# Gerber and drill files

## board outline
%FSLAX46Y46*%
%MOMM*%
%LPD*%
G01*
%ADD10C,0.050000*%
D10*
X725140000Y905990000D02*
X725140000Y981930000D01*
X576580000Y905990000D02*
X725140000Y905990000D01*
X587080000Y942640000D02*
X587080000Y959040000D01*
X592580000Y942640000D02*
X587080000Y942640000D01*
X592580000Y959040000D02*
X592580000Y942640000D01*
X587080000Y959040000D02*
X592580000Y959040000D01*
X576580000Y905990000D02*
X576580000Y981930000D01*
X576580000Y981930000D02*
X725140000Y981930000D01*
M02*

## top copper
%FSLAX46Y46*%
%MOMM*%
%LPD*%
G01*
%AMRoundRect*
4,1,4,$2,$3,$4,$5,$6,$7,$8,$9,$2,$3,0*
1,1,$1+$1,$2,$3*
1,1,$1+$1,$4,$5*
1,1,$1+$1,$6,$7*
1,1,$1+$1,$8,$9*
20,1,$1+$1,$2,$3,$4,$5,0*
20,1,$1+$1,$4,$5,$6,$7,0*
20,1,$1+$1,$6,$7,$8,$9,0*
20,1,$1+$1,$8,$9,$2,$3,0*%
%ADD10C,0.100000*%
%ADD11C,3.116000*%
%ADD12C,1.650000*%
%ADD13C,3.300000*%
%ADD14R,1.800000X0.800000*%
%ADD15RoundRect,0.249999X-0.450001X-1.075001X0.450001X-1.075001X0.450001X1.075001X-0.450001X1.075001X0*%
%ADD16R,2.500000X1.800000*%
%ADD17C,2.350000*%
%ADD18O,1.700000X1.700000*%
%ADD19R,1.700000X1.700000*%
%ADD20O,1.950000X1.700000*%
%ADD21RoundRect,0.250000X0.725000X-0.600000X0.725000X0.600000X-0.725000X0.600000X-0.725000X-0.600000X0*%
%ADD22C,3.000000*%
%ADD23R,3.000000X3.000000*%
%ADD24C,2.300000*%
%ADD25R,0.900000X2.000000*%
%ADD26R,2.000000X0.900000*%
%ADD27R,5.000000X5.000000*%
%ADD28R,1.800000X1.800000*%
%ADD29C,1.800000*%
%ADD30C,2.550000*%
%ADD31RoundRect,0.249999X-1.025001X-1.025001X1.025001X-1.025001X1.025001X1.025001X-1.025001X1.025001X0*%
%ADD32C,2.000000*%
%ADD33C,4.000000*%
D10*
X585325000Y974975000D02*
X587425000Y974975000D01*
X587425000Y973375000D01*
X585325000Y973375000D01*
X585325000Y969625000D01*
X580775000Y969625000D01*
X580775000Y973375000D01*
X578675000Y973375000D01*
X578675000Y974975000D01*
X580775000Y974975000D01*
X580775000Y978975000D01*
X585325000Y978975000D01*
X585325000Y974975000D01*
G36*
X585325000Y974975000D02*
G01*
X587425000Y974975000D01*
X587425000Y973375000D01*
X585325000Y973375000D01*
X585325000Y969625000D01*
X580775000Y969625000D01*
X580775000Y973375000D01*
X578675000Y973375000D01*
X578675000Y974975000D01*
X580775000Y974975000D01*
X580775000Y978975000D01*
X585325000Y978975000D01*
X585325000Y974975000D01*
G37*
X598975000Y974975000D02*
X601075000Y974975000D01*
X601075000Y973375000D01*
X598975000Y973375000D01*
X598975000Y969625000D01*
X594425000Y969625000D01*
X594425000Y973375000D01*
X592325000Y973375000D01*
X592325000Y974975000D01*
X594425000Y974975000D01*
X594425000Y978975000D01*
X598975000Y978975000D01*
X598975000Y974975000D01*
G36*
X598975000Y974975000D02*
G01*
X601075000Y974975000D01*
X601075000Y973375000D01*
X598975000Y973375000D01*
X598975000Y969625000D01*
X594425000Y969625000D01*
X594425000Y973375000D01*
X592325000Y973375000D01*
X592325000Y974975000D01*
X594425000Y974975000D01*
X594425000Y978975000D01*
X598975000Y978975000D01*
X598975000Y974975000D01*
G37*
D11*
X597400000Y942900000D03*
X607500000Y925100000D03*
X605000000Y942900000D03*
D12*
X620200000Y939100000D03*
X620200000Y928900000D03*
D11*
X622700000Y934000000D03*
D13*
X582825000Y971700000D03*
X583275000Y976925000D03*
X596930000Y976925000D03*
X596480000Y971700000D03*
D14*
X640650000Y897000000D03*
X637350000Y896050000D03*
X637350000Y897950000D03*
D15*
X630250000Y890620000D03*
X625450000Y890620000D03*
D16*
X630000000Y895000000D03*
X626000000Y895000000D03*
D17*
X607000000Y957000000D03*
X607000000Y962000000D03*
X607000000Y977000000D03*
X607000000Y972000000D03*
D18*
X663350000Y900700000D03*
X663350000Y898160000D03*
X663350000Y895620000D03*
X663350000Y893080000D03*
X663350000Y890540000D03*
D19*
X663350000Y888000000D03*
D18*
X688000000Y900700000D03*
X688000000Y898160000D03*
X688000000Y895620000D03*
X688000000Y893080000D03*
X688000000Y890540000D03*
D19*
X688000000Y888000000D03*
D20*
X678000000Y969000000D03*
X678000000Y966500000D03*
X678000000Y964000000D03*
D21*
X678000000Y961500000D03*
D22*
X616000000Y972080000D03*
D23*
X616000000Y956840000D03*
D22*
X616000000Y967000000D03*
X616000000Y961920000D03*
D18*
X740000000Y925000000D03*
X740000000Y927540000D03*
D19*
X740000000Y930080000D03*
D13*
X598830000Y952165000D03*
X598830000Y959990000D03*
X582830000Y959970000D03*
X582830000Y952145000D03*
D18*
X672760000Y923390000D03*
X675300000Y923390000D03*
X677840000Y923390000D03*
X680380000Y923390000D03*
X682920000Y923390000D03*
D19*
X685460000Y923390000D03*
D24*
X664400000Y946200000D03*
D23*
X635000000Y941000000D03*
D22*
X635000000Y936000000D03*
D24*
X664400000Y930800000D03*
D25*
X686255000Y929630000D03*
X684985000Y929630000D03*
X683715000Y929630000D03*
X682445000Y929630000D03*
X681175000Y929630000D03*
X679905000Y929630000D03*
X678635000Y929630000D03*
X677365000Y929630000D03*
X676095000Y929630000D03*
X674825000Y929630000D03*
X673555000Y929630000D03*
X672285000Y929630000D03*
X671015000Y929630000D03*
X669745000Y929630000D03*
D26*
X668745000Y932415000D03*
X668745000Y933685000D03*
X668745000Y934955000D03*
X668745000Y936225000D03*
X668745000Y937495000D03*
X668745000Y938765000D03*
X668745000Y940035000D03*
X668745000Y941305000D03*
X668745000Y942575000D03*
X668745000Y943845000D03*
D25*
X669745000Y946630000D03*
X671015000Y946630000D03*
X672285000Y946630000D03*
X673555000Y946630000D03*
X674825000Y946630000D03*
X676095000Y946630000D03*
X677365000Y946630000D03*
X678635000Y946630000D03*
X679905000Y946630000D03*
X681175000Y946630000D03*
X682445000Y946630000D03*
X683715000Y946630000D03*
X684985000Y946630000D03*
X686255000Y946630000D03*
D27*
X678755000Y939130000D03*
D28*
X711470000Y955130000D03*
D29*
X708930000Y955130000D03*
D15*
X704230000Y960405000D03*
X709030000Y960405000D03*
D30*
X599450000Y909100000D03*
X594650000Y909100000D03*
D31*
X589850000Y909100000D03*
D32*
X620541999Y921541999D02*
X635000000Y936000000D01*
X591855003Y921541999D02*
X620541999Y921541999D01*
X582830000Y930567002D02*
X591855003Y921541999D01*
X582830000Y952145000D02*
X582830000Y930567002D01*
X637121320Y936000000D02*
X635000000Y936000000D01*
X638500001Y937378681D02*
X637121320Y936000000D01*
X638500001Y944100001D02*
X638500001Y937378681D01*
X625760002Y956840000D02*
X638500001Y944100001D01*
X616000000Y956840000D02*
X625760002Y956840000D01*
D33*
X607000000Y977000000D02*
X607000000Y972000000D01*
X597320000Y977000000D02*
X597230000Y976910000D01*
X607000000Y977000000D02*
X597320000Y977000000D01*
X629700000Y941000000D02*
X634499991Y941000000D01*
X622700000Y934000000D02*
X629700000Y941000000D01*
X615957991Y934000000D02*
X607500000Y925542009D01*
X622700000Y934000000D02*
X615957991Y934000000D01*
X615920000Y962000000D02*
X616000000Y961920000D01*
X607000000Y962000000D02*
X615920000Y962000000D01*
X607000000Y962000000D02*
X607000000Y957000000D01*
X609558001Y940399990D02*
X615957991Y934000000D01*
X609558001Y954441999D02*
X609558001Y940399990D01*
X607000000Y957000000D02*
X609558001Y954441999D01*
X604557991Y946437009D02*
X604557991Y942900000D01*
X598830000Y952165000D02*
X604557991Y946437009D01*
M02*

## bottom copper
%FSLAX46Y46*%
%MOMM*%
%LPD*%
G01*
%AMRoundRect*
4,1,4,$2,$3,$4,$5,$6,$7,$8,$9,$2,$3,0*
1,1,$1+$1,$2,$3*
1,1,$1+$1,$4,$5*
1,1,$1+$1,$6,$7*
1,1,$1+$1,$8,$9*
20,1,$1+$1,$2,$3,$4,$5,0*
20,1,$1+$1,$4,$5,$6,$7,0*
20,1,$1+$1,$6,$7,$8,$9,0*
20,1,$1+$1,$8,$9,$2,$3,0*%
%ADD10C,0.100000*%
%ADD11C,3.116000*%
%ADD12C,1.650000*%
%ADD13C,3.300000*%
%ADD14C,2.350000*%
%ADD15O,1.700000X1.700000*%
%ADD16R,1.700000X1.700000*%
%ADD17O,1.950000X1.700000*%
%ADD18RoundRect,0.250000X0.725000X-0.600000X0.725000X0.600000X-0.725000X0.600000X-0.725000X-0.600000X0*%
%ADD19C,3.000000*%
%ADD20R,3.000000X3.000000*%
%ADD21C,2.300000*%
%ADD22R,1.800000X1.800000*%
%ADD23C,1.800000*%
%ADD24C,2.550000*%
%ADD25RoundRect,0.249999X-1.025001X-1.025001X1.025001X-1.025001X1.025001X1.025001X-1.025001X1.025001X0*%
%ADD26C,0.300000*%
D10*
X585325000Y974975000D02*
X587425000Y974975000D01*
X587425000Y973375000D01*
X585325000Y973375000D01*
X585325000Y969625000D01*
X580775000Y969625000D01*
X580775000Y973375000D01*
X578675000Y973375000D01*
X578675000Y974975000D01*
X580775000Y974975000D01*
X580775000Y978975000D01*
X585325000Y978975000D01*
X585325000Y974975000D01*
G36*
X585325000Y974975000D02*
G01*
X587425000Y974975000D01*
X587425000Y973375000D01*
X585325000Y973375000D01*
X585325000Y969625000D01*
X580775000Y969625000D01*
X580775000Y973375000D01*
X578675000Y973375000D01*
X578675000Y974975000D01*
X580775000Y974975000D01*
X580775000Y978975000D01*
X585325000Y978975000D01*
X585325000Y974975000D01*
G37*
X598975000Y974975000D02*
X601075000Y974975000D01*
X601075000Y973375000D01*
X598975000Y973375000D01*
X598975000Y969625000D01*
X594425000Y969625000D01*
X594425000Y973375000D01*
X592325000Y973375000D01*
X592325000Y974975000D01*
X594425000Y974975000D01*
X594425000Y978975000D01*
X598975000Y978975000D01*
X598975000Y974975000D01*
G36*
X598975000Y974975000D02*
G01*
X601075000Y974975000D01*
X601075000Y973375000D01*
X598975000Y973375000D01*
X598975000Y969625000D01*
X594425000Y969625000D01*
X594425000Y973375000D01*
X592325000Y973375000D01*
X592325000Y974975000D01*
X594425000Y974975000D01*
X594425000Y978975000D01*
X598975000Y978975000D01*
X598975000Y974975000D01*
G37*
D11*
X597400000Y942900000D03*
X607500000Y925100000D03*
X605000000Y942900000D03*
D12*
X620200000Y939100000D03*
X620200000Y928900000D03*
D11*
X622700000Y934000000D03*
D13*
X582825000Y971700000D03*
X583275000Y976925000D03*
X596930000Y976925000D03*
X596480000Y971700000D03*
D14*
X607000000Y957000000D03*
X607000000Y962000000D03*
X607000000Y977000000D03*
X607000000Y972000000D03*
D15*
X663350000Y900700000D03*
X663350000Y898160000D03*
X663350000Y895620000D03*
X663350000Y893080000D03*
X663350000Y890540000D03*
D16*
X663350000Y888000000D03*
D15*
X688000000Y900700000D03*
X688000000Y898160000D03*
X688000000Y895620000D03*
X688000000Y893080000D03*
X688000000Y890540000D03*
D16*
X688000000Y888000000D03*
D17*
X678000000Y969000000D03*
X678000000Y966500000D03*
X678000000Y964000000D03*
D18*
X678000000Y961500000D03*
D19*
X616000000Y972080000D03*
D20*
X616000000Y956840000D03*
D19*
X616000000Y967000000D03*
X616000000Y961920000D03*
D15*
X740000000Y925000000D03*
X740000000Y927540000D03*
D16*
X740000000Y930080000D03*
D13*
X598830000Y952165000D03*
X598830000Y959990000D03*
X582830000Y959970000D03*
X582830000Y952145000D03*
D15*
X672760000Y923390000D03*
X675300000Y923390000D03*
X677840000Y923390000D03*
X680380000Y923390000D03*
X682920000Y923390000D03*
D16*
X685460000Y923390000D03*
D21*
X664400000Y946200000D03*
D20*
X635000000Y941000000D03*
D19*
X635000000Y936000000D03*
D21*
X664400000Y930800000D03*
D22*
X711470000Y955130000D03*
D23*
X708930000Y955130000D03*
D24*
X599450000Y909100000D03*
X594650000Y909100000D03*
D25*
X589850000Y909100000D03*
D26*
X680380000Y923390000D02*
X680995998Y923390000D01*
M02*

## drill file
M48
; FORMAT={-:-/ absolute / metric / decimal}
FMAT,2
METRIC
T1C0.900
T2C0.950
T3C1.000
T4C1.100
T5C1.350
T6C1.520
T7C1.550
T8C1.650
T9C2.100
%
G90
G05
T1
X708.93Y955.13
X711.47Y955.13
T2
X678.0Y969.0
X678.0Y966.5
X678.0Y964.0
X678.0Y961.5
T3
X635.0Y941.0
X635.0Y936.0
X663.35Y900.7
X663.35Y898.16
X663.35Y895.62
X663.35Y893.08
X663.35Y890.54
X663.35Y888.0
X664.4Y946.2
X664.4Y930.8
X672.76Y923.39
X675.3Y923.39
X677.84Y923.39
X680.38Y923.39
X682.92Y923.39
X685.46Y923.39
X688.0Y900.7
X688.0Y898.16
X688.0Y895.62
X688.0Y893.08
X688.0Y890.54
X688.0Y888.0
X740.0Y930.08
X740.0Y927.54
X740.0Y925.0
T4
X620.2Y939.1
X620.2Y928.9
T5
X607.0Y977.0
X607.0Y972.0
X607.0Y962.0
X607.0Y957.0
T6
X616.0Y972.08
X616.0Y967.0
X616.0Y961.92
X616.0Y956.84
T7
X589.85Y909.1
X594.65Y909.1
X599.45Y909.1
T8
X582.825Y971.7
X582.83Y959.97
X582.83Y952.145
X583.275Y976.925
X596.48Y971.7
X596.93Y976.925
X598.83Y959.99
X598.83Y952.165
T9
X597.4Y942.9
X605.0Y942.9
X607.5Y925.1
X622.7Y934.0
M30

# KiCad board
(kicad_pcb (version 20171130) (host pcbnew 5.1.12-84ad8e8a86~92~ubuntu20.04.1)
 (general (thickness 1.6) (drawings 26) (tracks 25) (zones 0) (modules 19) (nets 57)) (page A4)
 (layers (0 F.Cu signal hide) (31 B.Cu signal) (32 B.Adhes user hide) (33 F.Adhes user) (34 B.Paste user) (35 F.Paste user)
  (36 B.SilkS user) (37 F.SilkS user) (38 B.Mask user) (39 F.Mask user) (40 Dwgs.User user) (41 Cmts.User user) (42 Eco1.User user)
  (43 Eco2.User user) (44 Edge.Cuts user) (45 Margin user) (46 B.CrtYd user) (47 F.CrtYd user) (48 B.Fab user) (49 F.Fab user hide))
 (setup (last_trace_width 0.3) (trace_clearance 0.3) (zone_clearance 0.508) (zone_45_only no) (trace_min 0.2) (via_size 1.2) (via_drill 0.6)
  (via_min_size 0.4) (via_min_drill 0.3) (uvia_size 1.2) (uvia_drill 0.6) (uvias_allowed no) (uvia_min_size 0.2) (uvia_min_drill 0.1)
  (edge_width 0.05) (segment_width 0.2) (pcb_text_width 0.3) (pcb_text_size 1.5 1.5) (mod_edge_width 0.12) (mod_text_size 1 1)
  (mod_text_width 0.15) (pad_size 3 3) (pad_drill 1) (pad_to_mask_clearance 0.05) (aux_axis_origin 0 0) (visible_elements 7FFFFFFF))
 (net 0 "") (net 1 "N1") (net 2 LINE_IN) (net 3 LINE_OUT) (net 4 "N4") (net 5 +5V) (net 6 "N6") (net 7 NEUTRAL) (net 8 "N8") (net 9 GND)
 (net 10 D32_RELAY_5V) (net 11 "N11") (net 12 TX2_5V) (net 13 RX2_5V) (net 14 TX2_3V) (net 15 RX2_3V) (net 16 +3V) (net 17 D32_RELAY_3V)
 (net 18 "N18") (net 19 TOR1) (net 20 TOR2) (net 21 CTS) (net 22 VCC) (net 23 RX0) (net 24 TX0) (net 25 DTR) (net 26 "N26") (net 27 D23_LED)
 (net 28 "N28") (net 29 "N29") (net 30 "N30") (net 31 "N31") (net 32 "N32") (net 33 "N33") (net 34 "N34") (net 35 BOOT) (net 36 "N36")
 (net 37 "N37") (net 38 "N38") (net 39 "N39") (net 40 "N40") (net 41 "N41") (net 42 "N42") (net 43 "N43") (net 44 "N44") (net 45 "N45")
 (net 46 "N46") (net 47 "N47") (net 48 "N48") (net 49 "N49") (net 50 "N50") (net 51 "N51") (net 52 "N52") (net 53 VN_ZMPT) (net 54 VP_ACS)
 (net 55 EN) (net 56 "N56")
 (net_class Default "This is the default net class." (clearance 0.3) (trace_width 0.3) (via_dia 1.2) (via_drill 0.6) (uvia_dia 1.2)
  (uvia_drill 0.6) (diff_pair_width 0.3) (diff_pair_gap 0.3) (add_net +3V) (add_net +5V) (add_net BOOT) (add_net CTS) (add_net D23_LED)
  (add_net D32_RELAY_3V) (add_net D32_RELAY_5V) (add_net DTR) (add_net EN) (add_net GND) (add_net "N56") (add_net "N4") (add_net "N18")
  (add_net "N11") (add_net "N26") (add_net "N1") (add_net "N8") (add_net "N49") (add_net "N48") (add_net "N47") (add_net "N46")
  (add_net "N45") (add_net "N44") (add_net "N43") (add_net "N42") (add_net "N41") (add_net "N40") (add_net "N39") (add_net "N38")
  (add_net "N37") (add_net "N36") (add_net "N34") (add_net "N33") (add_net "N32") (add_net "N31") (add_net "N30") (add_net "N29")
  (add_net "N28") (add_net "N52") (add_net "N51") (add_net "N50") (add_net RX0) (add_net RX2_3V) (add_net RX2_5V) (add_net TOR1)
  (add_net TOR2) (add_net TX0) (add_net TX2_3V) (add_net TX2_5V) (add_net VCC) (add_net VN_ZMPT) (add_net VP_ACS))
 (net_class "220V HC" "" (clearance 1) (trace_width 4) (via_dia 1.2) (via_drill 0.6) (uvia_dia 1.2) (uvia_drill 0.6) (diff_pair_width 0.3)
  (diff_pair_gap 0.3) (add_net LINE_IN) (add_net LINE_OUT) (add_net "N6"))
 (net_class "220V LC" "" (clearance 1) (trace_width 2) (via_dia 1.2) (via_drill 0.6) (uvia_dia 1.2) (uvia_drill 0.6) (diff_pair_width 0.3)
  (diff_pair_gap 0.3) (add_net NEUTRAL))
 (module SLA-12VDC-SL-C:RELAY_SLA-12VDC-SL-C (layer F.Cu) (at 605 -934 90)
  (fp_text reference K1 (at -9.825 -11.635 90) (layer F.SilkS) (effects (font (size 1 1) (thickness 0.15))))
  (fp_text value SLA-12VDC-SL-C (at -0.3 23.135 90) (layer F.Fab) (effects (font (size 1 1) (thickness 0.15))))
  (pad NC thru_hole circle (at 8.9 -7.6 90) (size 3.116 3.116) (drill 2.1) (layers *.Cu *.Mask) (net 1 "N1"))
  (pad COM2 thru_hole circle (at -8.9 2.5 90) (size 3.116 3.116) (drill 2.1) (layers *.Cu *.Mask) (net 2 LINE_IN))
  (pad NO thru_hole circle (at 8.9 0 90) (size 3.116 3.116) (drill 2.1) (layers *.Cu *.Mask) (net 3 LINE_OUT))
  (pad C2 thru_hole circle (at 5.1 15.2 90) (size 1.65 1.65) (drill 1.1) (layers *.Cu *.Mask) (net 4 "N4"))
  (pad C1 thru_hole circle (at -5.1 15.2 90) (size 1.65 1.65) (drill 1.1) (layers *.Cu *.Mask) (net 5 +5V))
  (pad COM1 thru_hole circle (at 0 17.7 90) (size 3.116 3.116) (drill 2.1) (layers *.Cu *.Mask) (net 2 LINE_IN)))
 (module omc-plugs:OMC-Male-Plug (layer F.Cu) (at 583 -974)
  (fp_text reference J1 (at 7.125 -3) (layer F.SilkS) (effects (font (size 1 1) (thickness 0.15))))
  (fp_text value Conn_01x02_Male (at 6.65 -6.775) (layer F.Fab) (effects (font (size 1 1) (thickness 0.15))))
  (fp_poly
   (pts (xy 2.325 -0.975) (xy 4.425 -0.975) (xy 4.425 0.625) (xy 2.325 0.625) (xy 2.325 4.375) (xy -2.225 4.375) (xy -2.225 0.625)
    (xy -4.325 0.625) (xy -4.325 -0.975) (xy -2.225 -0.975) (xy -2.225 -4.975) (xy 2.325 -4.975))
   (layer F.Cu) (width 0.1))
  (fp_poly
   (pts (xy 2.325 -0.975) (xy 4.425 -0.975) (xy 4.425 0.625) (xy 2.325 0.625) (xy 2.325 4.375) (xy -2.225 4.375) (xy -2.225 0.625)
    (xy -4.325 0.625) (xy -4.325 -0.975) (xy -2.225 -0.975) (xy -2.225 -4.975) (xy 2.325 -4.975))
   (layer B.Cu) (width 0.1))
  (fp_poly
   (pts (xy 15.975 -0.975) (xy 18.075 -0.975) (xy 18.075 0.625) (xy 15.975 0.625) (xy 15.975 4.375) (xy 11.425 4.375) (xy 11.425 0.625)
    (xy 9.325 0.625) (xy 9.325 -0.975) (xy 11.425 -0.975) (xy 11.425 -4.975) (xy 15.975 -4.975))
   (layer B.Cu) (width 0.1))
  (fp_poly
   (pts (xy 15.975 -0.975) (xy 18.075 -0.975) (xy 18.075 0.625) (xy 15.975 0.625) (xy 15.975 4.375) (xy 11.425 4.375) (xy 11.425 0.625)
    (xy 9.325 0.625) (xy 9.325 -0.975) (xy 11.425 -0.975) (xy 11.425 -4.975) (xy 15.975 -4.975))
   (layer F.Cu) (width 0.1))
  (pad 1 thru_hole circle (at -0.175 2.3) (size 3.3 3.3) (drill 1.65) (layers *.Cu *.Mask) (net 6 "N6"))
  (pad 1 thru_hole circle (at 0.275 -2.925 270) (size 3.3 3.3) (drill 1.65) (layers *.Cu *.Mask) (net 6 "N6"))
  (pad 2 thru_hole circle (at 13.93 -2.925 270) (size 3.3 3.3) (drill 1.65) (layers *.Cu *.Mask) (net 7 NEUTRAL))
  (pad 2 thru_hole circle (at 13.48 2.3) (size 3.3 3.3) (drill 1.65) (layers *.Cu *.Mask) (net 7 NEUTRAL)))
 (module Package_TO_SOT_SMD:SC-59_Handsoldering (layer F.Cu) (at 639 -897)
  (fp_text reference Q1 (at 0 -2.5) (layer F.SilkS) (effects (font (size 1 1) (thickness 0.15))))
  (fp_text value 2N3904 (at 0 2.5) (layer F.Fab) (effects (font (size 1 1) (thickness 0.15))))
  (pad 3 smd rect (at 1.65 0) (size 1.8 0.8) (layers F.Cu F.Paste F.Mask) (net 4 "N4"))
  (pad 2 smd rect (at -1.65 0.95) (size 1.8 0.8) (layers F.Cu F.Paste F.Mask) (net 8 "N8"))
  (pad 1 smd rect (at -1.65 -0.95) (size 1.8 0.8) (layers F.Cu F.Paste F.Mask) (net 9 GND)))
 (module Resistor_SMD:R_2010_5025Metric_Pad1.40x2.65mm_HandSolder (layer F.Cu) (at 627.85 -890.62)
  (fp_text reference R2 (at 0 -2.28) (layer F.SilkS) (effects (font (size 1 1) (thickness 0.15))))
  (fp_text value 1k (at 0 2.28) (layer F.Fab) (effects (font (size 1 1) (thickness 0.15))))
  (pad 2 smd roundrect (at 2.4 0) (size 1.4 2.65) (layers F.Cu F.Paste F.Mask) (roundrect_rratio 0.178571) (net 8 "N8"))
  (pad 1 smd roundrect (at -2.4 0) (size 1.4 2.65) (layers F.Cu F.Paste F.Mask) (roundrect_rratio 0.178571) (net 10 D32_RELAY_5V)))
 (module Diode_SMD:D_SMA (layer F.Cu) (at 628 -895)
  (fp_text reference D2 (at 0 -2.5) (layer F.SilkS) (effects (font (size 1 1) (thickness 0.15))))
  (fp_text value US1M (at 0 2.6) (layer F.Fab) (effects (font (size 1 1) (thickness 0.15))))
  (pad 2 smd rect (at 2 0) (size 2.5 1.8) (layers F.Cu F.Paste F.Mask) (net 4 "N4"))
  (pad 1 smd rect (at -2 0) (size 2.5 1.8) (layers F.Cu F.Paste F.Mask) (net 5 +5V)))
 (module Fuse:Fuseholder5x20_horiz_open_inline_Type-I (layer F.Cu) (at 607 -957 90)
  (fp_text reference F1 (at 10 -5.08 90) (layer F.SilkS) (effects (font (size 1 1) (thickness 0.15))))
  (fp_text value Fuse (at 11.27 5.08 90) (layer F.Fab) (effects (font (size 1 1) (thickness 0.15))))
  (pad 1 thru_hole circle (at 0 0 90) (size 2.35 2.35) (drill 1.35) (layers *.Cu *.Mask) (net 2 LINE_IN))
  (pad 1 thru_hole circle (at 5 0 90) (size 2.35 2.35) (drill 1.35) (layers *.Cu *.Mask) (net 2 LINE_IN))
  (pad 2 thru_hole circle (at 20 0 90) (size 2.35 2.35) (drill 1.35) (layers *.Cu *.Mask) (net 6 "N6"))
  (pad 2 thru_hole circle (at 15 0 90) (size 2.35 2.35) (drill 1.35) (layers *.Cu *.Mask) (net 6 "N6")))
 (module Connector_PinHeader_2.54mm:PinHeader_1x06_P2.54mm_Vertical (layer F.Cu) (at 663.35 -888 180)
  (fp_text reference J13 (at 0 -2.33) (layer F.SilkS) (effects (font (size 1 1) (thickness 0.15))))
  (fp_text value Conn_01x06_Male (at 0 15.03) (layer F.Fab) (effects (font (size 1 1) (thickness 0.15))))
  (pad 6 thru_hole oval (at 0 12.7 180) (size 1.7 1.7) (drill 1) (layers *.Cu *.Mask) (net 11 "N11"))
  (pad 5 thru_hole oval (at 0 10.16 180) (size 1.7 1.7) (drill 1) (layers *.Cu *.Mask) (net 10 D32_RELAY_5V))
  (pad 4 thru_hole oval (at 0 7.62 180) (size 1.7 1.7) (drill 1) (layers *.Cu *.Mask) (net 9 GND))
  (pad 3 thru_hole oval (at 0 5.08 180) (size 1.7 1.7) (drill 1) (layers *.Cu *.Mask) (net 5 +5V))
  (pad 2 thru_hole oval (at 0 2.54 180) (size 1.7 1.7) (drill 1) (layers *.Cu *.Mask) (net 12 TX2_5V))
  (pad 1 thru_hole rect (at 0 0 180) (size 1.7 1.7) (drill 1) (layers *.Cu *.Mask) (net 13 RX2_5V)))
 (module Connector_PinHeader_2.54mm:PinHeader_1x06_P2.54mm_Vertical (layer F.Cu) (at 688 -888 180)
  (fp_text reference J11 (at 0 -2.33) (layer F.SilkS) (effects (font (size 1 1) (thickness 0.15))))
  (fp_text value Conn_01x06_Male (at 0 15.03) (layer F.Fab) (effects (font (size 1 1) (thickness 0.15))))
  (pad 6 thru_hole oval (at 0 12.7 180) (size 1.7 1.7) (drill 1) (layers *.Cu *.Mask) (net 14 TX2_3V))
  (pad 5 thru_hole oval (at 0 10.16 180) (size 1.7 1.7) (drill 1) (layers *.Cu *.Mask) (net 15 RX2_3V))
  (pad 4 thru_hole oval (at 0 7.62 180) (size 1.7 1.7) (drill 1) (layers *.Cu *.Mask) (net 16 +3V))
  (pad 3 thru_hole oval (at 0 5.08 180) (size 1.7 1.7) (drill 1) (layers *.Cu *.Mask) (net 9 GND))
  (pad 2 thru_hole oval (at 0 2.54 180) (size 1.7 1.7) (drill 1) (layers *.Cu *.Mask) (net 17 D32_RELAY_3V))
  (pad 1 thru_hole rect (at 0 0 180) (size 1.7 1.7) (drill 1) (layers *.Cu *.Mask) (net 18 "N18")))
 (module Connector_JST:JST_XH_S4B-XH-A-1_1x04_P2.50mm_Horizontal (layer F.Cu) (at 678 -961.5 90)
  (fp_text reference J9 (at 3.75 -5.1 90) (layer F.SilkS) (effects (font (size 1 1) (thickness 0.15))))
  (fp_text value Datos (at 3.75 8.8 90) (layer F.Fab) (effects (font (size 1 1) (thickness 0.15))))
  (pad 4 thru_hole oval (at 7.5 0 90) (size 1.7 1.95) (drill 0.95) (layers *.Cu *.Mask) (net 9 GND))
  (pad 3 thru_hole oval (at 5 0 90) (size 1.7 1.95) (drill 0.95) (layers *.Cu *.Mask) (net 12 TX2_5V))
  (pad 2 thru_hole oval (at 2.5 0 90) (size 1.7 1.95) (drill 0.95) (layers *.Cu *.Mask) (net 13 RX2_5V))
  (pad 1 thru_hole roundrect (at 0 0 90) (size 1.7 1.95) (drill 0.95) (layers *.Cu *.Mask) (roundrect_rratio 0.147059) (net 5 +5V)))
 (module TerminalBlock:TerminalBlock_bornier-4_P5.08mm (layer F.Cu) (at 616 -956.84 90)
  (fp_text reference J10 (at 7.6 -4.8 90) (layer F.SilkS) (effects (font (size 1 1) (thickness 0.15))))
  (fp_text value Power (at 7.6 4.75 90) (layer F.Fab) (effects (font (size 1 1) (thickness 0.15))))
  (pad 4 thru_hole circle (at 15.24 0 90) (size 3 3) (drill 1.52) (layers *.Cu *.Mask) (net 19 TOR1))
  (pad 1 thru_hole rect (at 0 0 90) (size 3 3) (drill 1.52) (layers *.Cu *.Mask) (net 7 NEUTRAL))
  (pad 3 thru_hole circle (at 10.16 0 90) (size 3 3) (drill 1.52) (layers *.Cu *.Mask) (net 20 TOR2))
  (pad 2 thru_hole circle (at 5.08 0 90) (size 3 3) (drill 1.52) (layers *.Cu *.Mask) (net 2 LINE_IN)))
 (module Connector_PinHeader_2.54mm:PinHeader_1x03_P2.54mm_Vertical (layer F.Cu) (at 740 -930.08)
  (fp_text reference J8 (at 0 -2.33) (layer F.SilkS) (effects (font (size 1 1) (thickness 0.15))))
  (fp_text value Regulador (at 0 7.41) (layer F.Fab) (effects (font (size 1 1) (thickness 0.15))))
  (pad 3 thru_hole oval (at 0 5.08) (size 1.7 1.7) (drill 1) (layers *.Cu *.Mask) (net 5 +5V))
  (pad 2 thru_hole oval (at 0 2.54) (size 1.7 1.7) (drill 1) (layers *.Cu *.Mask) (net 16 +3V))
  (pad 1 thru_hole rect (at 0 0) (size 1.7 1.7) (drill 1) (layers *.Cu *.Mask) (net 9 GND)))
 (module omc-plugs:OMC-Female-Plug (layer F.Cu) (at 598.18 -956.04)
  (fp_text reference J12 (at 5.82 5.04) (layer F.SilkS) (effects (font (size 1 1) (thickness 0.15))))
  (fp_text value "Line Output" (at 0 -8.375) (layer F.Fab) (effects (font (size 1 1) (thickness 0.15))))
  (pad 1 thru_hole circle (at 0.65 3.875) (size 3.3 3.3) (drill 1.65) (layers *.Cu *.Mask) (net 3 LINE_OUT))
  (pad 1 thru_hole circle (at 0.65 -3.95) (size 3.3 3.3) (drill 1.65) (layers *.Cu *.Mask) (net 3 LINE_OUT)))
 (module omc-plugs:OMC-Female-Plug (layer F.Cu) (at 582.18 -956.02)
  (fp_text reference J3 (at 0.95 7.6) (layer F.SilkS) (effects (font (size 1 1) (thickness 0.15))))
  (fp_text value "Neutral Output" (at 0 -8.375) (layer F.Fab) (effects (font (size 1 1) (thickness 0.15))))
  (pad 1 thru_hole circle (at 0.65 -3.95) (size 3.3 3.3) (drill 1.65) (layers *.Cu *.Mask) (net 7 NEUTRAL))
  (pad 1 thru_hole circle (at 0.65 3.875) (size 3.3 3.3) (drill 1.65) (layers *.Cu *.Mask) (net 7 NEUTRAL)))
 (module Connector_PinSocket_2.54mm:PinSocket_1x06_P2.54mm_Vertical (layer F.Cu) (at 685.46 -923.39 270)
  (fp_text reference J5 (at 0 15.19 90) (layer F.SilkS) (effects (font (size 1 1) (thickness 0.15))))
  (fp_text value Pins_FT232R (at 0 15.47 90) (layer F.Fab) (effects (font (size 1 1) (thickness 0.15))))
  (pad 6 thru_hole oval (at 0 12.7 270) (size 1.7 1.7) (drill 1) (layers *.Cu *.Mask) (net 9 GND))
  (pad 5 thru_hole oval (at 0 10.16 270) (size 1.7 1.7) (drill 1) (layers *.Cu *.Mask) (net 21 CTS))
  (pad 4 thru_hole oval (at 0 7.62 270) (size 1.7 1.7) (drill 1) (layers *.Cu *.Mask) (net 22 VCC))
  (pad 3 thru_hole oval (at 0 5.08 270) (size 1.7 1.7) (drill 1) (layers *.Cu *.Mask) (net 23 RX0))
  (pad 2 thru_hole oval (at 0 2.54 270) (size 1.7 1.7) (drill 1) (layers *.Cu *.Mask) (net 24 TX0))
  (pad 1 thru_hole rect (at 0 0 270) (size 1.7 1.7) (drill 1) (layers *.Cu *.Mask) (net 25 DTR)))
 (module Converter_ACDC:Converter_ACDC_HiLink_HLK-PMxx (layer F.Cu) (at 635 -941)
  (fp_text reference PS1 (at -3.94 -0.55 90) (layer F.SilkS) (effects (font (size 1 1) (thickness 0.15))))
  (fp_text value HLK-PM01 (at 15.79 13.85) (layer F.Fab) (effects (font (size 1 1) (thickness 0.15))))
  (pad 3 thru_hole circle (at 29.4 -5.2) (size 2.3 2.3) (drill 1) (layers *.Cu *.Mask) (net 9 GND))
  (pad 1 thru_hole rect (at 0 0) (size 3 3) (drill 1) (layers *.Cu *.Mask) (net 2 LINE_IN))
  (pad 2 thru_hole circle (at 0 5) (size 3 3) (drill 1) (layers *.Cu *.Mask) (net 7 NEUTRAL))
  (pad 4 thru_hole circle (at 29.4 10.2) (size 2.3 2.3) (drill 1) (layers *.Cu *.Mask) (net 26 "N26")))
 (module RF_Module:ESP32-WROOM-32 (layer F.Cu) (at 678 -938.13 270)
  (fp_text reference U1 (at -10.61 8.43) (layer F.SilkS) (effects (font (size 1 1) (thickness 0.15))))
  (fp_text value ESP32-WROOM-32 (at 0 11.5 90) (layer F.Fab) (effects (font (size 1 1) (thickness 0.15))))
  (pad 38 smd rect (at 8.5 -8.255 270) (size 2 0.9) (layers F.Cu F.Paste F.Mask) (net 9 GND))
  (pad 37 smd rect (at 8.5 -6.985 270) (size 2 0.9) (layers F.Cu F.Paste F.Mask) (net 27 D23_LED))
  (pad 36 smd rect (at 8.5 -5.715 270) (size 2 0.9) (layers F.Cu F.Paste F.Mask) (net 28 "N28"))
  (pad 35 smd rect (at 8.5 -4.445 270) (size 2 0.9) (layers F.Cu F.Paste F.Mask) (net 24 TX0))
  (pad 34 smd rect (at 8.5 -3.175 270) (size 2 0.9) (layers F.Cu F.Paste F.Mask) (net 23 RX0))
  (pad 33 smd rect (at 8.5 -1.905 270) (size 2 0.9) (layers F.Cu F.Paste F.Mask) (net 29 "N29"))
  (pad 32 smd rect (at 8.5 -0.635 270) (size 2 0.9) (layers F.Cu F.Paste F.Mask) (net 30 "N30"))
  (pad 31 smd rect (at 8.5 0.635 270) (size 2 0.9) (layers F.Cu F.Paste F.Mask) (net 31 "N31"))
  (pad 30 smd rect (at 8.5 1.905 270) (size 2 0.9) (layers F.Cu F.Paste F.Mask) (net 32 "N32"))
  (pad 29 smd rect (at 8.5 3.175 270) (size 2 0.9) (layers F.Cu F.Paste F.Mask) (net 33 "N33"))
  (pad 28 smd rect (at 8.5 4.445 270) (size 2 0.9) (layers F.Cu F.Paste F.Mask) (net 14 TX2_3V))
  (pad 27 smd rect (at 8.5 5.715 270) (size 2 0.9) (layers F.Cu F.Paste F.Mask) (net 15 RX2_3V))
  (pad 26 smd rect (at 8.5 6.985 270) (size 2 0.9) (layers F.Cu F.Paste F.Mask) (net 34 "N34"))
  (pad 25 smd rect (at 8.5 8.255 270) (size 2 0.9) (layers F.Cu F.Paste F.Mask) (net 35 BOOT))
  (pad 24 smd rect (at 5.715 9.255) (size 2 0.9) (layers F.Cu F.Paste F.Mask) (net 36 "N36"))
  (pad 23 smd rect (at 4.445 9.255) (size 2 0.9) (layers F.Cu F.Paste F.Mask) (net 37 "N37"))
  (pad 22 smd rect (at 3.175 9.255) (size 2 0.9) (layers F.Cu F.Paste F.Mask) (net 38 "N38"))
  (pad 21 smd rect (at 1.905 9.255) (size 2 0.9) (layers F.Cu F.Paste F.Mask) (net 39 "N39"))
  (pad 20 smd rect (at 0.635 9.255) (size 2 0.9) (layers F.Cu F.Paste F.Mask) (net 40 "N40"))
  (pad 19 smd rect (at -0.635 9.255) (size 2 0.9) (layers F.Cu F.Paste F.Mask) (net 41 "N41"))
  (pad 18 smd rect (at -1.905 9.255) (size 2 0.9) (layers F.Cu F.Paste F.Mask) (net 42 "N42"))
  (pad 17 smd rect (at -3.175 9.255) (size 2 0.9) (layers F.Cu F.Paste F.Mask) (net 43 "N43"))
  (pad 16 smd rect (at -4.445 9.255) (size 2 0.9) (layers F.Cu F.Paste F.Mask) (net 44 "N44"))
  (pad 15 smd rect (at -5.715 9.255) (size 2 0.9) (layers F.Cu F.Paste F.Mask) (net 9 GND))
  (pad 14 smd rect (at -8.5 8.255 270) (size 2 0.9) (layers F.Cu F.Paste F.Mask) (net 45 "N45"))
  (pad 13 smd rect (at -8.5 6.985 270) (size 2 0.9) (layers F.Cu F.Paste F.Mask) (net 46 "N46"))
  (pad 12 smd rect (at -8.5 5.715 270) (size 2 0.9) (layers F.Cu F.Paste F.Mask) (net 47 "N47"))
  (pad 11 smd rect (at -8.5 4.445 270) (size 2 0.9) (layers F.Cu F.Paste F.Mask) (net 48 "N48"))
  (pad 10 smd rect (at -8.5 3.175 270) (size 2 0.9) (layers F.Cu F.Paste F.Mask) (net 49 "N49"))
  (pad 9 smd rect (at -8.5 1.905 270) (size 2 0.9) (layers F.Cu F.Paste F.Mask) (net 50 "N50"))
  (pad 8 smd rect (at -8.5 0.635 270) (size 2 0.9) (layers F.Cu F.Paste F.Mask) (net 17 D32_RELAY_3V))
  (pad 7 smd rect (at -8.5 -0.635 270) (size 2 0.9) (layers F.Cu F.Paste F.Mask) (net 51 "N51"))
  (pad 6 smd rect (at -8.5 -1.905 270) (size 2 0.9) (layers F.Cu F.Paste F.Mask) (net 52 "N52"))
  (pad 5 smd rect (at -8.5 -3.175 270) (size 2 0.9) (layers F.Cu F.Paste F.Mask) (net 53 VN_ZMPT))
  (pad 4 smd rect (at -8.5 -4.445 270) (size 2 0.9) (layers F.Cu F.Paste F.Mask) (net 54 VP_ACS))
  (pad 3 smd rect (at -8.5 -5.715 270) (size 2 0.9) (layers F.Cu F.Paste F.Mask) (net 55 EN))
  (pad 2 smd rect (at -8.5 -6.985 270) (size 2 0.9) (layers F.Cu F.Paste F.Mask) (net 16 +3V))
  (pad 1 smd rect (at -8.5 -8.255 270) (size 2 0.9) (layers F.Cu F.Paste F.Mask) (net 9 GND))
  (pad 39 smd rect (at -1 -0.755 270) (size 5 5) (layers F.Cu F.Paste F.Mask) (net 9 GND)))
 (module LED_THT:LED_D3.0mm (layer F.Cu) (at 711.47 -955.13 180)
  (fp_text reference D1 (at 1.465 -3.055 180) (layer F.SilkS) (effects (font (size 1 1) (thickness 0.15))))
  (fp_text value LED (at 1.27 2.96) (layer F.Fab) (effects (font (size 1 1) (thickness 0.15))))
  (pad 1 thru_hole rect (at 0 0 180) (size 1.8 1.8) (drill 0.9) (layers *.Cu *.Mask) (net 9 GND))
  (pad 2 thru_hole circle (at 2.54 0 180) (size 1.8 1.8) (drill 0.9) (layers *.Cu *.Mask) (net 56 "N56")))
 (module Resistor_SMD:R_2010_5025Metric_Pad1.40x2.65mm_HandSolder (layer F.Cu) (at 706.63 -960.405)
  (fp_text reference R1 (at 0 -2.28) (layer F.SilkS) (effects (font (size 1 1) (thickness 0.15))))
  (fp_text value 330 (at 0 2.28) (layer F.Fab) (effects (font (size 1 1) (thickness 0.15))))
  (pad 1 smd roundrect (at -2.4 0) (size 1.4 2.65) (layers F.Cu F.Paste F.Mask) (roundrect_rratio 0.1785707142857143) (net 27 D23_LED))
  (pad 2 smd roundrect (at 2.4 0) (size 1.4 2.65) (layers F.Cu F.Paste F.Mask) (roundrect_rratio 0.1785707142857143) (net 56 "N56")))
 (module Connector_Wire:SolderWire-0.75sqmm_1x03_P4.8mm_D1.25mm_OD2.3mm (layer F.Cu) (at 589.85 -909.1)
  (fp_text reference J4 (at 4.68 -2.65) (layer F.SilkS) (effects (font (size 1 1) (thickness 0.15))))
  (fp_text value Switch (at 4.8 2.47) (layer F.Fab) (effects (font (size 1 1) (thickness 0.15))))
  (pad 3 thru_hole circle (at 9.6 0) (size 2.55 2.55) (drill 1.55) (layers *.Cu *.Mask) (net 9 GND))
  (pad 2 thru_hole circle (at 4.8 0) (size 2.55 2.55) (drill 1.55) (layers *.Cu *.Mask) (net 5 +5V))
  (pad 1 thru_hole roundrect (at 0 0) (size 2.55 2.55) (drill 1.55) (layers *.Cu *.Mask) (roundrect_rratio 0.09803882352941176)
   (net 26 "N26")))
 (gr_line (start 725.14 -905.99) (end 725.14 -981.93) (layer Edge.Cuts) (width 0.05))
 (gr_line (start 576.58 -905.99) (end 725.14 -905.99) (layer Edge.Cuts) (width 0.05))
 (gr_line (start 587.08 -942.64) (end 587.08 -959.04) (layer Edge.Cuts) (width 0.05))
 (gr_line (start 592.58 -942.64) (end 587.08 -942.64) (layer Edge.Cuts) (width 0.05))
 (gr_line (start 592.58 -959.04) (end 592.58 -942.64) (layer Edge.Cuts) (width 0.05))
 (gr_line (start 587.08 -959.04) (end 592.58 -959.04) (layer Edge.Cuts) (width 0.05))
 (gr_line (start 576.58 -905.99) (end 576.58 -981.93) (layer Edge.Cuts) (width 0.05))
 (gr_line (start 576.58 -981.93) (end 725.14 -981.93) (layer Edge.Cuts) (width 0.05))
 (segment (start 680.38 -923.39) (end 680.995998 -923.39) (width 0.3) (layer B.Cu) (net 23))
 (segment (start 620.541999 -921.541999) (end 635 -936) (width 2) (layer F.Cu) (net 7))
 (segment (start 591.855003 -921.541999) (end 620.541999 -921.541999) (width 2) (layer F.Cu) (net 7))
 (segment (start 582.83 -930.567002) (end 591.855003 -921.541999) (width 2) (layer F.Cu) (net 7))
 (segment (start 582.83 -952.145) (end 582.83 -930.567002) (width 2) (layer F.Cu) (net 7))
 (segment (start 637.12132 -936) (end 635 -936) (width 2) (layer F.Cu) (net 7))
 (segment (start 638.500001 -937.378681) (end 637.12132 -936) (width 2) (layer F.Cu) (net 7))
 (segment (start 638.500001 -944.100001) (end 638.500001 -937.378681) (width 2) (layer F.Cu) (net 7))
 (segment (start 625.760002 -956.84) (end 638.500001 -944.100001) (width 2) (layer F.Cu) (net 7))
 (segment (start 616 -956.84) (end 625.760002 -956.84) (width 2) (layer F.Cu) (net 7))
 (segment (start 607 -977) (end 607 -972) (width 4) (layer F.Cu) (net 6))
 (segment (start 597.32 -977) (end 597.23 -976.91) (width 4) (layer F.Cu) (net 6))
 (segment (start 607 -977) (end 597.32 -977) (width 4) (layer F.Cu) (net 6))
 (segment (start 629.7 -941) (end 634.499991 -941) (width 4) (layer F.Cu) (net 2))
 (segment (start 622.7 -934) (end 629.7 -941) (width 4) (layer F.Cu) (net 2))
 (segment (start 615.957991 -934) (end 607.5 -925.542009) (width 4) (layer F.Cu) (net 2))
 (segment (start 622.7 -934) (end 615.957991 -934) (width 4) (layer F.Cu) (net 2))
 (segment (start 615.92 -962) (end 616 -961.92) (width 4) (layer F.Cu) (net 2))
 (segment (start 607 -962) (end 615.92 -962) (width 4) (layer F.Cu) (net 2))
 (segment (start 607 -962) (end 607 -957) (width 4) (layer F.Cu) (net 2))
 (segment (start 609.558001 -940.39999) (end 615.957991 -934) (width 4) (layer F.Cu) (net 2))
 (segment (start 609.558001 -954.441999) (end 609.558001 -940.39999) (width 4) (layer F.Cu) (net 2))
 (segment (start 607 -957) (end 609.558001 -954.441999) (width 4) (layer F.Cu) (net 2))
 (segment (start 604.557991 -946.437009) (end 604.557991 -942.9) (width 4) (layer F.Cu) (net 3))
 (segment (start 598.83 -952.165) (end 604.557991 -946.437009) (width 4) (layer F.Cu) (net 3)))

